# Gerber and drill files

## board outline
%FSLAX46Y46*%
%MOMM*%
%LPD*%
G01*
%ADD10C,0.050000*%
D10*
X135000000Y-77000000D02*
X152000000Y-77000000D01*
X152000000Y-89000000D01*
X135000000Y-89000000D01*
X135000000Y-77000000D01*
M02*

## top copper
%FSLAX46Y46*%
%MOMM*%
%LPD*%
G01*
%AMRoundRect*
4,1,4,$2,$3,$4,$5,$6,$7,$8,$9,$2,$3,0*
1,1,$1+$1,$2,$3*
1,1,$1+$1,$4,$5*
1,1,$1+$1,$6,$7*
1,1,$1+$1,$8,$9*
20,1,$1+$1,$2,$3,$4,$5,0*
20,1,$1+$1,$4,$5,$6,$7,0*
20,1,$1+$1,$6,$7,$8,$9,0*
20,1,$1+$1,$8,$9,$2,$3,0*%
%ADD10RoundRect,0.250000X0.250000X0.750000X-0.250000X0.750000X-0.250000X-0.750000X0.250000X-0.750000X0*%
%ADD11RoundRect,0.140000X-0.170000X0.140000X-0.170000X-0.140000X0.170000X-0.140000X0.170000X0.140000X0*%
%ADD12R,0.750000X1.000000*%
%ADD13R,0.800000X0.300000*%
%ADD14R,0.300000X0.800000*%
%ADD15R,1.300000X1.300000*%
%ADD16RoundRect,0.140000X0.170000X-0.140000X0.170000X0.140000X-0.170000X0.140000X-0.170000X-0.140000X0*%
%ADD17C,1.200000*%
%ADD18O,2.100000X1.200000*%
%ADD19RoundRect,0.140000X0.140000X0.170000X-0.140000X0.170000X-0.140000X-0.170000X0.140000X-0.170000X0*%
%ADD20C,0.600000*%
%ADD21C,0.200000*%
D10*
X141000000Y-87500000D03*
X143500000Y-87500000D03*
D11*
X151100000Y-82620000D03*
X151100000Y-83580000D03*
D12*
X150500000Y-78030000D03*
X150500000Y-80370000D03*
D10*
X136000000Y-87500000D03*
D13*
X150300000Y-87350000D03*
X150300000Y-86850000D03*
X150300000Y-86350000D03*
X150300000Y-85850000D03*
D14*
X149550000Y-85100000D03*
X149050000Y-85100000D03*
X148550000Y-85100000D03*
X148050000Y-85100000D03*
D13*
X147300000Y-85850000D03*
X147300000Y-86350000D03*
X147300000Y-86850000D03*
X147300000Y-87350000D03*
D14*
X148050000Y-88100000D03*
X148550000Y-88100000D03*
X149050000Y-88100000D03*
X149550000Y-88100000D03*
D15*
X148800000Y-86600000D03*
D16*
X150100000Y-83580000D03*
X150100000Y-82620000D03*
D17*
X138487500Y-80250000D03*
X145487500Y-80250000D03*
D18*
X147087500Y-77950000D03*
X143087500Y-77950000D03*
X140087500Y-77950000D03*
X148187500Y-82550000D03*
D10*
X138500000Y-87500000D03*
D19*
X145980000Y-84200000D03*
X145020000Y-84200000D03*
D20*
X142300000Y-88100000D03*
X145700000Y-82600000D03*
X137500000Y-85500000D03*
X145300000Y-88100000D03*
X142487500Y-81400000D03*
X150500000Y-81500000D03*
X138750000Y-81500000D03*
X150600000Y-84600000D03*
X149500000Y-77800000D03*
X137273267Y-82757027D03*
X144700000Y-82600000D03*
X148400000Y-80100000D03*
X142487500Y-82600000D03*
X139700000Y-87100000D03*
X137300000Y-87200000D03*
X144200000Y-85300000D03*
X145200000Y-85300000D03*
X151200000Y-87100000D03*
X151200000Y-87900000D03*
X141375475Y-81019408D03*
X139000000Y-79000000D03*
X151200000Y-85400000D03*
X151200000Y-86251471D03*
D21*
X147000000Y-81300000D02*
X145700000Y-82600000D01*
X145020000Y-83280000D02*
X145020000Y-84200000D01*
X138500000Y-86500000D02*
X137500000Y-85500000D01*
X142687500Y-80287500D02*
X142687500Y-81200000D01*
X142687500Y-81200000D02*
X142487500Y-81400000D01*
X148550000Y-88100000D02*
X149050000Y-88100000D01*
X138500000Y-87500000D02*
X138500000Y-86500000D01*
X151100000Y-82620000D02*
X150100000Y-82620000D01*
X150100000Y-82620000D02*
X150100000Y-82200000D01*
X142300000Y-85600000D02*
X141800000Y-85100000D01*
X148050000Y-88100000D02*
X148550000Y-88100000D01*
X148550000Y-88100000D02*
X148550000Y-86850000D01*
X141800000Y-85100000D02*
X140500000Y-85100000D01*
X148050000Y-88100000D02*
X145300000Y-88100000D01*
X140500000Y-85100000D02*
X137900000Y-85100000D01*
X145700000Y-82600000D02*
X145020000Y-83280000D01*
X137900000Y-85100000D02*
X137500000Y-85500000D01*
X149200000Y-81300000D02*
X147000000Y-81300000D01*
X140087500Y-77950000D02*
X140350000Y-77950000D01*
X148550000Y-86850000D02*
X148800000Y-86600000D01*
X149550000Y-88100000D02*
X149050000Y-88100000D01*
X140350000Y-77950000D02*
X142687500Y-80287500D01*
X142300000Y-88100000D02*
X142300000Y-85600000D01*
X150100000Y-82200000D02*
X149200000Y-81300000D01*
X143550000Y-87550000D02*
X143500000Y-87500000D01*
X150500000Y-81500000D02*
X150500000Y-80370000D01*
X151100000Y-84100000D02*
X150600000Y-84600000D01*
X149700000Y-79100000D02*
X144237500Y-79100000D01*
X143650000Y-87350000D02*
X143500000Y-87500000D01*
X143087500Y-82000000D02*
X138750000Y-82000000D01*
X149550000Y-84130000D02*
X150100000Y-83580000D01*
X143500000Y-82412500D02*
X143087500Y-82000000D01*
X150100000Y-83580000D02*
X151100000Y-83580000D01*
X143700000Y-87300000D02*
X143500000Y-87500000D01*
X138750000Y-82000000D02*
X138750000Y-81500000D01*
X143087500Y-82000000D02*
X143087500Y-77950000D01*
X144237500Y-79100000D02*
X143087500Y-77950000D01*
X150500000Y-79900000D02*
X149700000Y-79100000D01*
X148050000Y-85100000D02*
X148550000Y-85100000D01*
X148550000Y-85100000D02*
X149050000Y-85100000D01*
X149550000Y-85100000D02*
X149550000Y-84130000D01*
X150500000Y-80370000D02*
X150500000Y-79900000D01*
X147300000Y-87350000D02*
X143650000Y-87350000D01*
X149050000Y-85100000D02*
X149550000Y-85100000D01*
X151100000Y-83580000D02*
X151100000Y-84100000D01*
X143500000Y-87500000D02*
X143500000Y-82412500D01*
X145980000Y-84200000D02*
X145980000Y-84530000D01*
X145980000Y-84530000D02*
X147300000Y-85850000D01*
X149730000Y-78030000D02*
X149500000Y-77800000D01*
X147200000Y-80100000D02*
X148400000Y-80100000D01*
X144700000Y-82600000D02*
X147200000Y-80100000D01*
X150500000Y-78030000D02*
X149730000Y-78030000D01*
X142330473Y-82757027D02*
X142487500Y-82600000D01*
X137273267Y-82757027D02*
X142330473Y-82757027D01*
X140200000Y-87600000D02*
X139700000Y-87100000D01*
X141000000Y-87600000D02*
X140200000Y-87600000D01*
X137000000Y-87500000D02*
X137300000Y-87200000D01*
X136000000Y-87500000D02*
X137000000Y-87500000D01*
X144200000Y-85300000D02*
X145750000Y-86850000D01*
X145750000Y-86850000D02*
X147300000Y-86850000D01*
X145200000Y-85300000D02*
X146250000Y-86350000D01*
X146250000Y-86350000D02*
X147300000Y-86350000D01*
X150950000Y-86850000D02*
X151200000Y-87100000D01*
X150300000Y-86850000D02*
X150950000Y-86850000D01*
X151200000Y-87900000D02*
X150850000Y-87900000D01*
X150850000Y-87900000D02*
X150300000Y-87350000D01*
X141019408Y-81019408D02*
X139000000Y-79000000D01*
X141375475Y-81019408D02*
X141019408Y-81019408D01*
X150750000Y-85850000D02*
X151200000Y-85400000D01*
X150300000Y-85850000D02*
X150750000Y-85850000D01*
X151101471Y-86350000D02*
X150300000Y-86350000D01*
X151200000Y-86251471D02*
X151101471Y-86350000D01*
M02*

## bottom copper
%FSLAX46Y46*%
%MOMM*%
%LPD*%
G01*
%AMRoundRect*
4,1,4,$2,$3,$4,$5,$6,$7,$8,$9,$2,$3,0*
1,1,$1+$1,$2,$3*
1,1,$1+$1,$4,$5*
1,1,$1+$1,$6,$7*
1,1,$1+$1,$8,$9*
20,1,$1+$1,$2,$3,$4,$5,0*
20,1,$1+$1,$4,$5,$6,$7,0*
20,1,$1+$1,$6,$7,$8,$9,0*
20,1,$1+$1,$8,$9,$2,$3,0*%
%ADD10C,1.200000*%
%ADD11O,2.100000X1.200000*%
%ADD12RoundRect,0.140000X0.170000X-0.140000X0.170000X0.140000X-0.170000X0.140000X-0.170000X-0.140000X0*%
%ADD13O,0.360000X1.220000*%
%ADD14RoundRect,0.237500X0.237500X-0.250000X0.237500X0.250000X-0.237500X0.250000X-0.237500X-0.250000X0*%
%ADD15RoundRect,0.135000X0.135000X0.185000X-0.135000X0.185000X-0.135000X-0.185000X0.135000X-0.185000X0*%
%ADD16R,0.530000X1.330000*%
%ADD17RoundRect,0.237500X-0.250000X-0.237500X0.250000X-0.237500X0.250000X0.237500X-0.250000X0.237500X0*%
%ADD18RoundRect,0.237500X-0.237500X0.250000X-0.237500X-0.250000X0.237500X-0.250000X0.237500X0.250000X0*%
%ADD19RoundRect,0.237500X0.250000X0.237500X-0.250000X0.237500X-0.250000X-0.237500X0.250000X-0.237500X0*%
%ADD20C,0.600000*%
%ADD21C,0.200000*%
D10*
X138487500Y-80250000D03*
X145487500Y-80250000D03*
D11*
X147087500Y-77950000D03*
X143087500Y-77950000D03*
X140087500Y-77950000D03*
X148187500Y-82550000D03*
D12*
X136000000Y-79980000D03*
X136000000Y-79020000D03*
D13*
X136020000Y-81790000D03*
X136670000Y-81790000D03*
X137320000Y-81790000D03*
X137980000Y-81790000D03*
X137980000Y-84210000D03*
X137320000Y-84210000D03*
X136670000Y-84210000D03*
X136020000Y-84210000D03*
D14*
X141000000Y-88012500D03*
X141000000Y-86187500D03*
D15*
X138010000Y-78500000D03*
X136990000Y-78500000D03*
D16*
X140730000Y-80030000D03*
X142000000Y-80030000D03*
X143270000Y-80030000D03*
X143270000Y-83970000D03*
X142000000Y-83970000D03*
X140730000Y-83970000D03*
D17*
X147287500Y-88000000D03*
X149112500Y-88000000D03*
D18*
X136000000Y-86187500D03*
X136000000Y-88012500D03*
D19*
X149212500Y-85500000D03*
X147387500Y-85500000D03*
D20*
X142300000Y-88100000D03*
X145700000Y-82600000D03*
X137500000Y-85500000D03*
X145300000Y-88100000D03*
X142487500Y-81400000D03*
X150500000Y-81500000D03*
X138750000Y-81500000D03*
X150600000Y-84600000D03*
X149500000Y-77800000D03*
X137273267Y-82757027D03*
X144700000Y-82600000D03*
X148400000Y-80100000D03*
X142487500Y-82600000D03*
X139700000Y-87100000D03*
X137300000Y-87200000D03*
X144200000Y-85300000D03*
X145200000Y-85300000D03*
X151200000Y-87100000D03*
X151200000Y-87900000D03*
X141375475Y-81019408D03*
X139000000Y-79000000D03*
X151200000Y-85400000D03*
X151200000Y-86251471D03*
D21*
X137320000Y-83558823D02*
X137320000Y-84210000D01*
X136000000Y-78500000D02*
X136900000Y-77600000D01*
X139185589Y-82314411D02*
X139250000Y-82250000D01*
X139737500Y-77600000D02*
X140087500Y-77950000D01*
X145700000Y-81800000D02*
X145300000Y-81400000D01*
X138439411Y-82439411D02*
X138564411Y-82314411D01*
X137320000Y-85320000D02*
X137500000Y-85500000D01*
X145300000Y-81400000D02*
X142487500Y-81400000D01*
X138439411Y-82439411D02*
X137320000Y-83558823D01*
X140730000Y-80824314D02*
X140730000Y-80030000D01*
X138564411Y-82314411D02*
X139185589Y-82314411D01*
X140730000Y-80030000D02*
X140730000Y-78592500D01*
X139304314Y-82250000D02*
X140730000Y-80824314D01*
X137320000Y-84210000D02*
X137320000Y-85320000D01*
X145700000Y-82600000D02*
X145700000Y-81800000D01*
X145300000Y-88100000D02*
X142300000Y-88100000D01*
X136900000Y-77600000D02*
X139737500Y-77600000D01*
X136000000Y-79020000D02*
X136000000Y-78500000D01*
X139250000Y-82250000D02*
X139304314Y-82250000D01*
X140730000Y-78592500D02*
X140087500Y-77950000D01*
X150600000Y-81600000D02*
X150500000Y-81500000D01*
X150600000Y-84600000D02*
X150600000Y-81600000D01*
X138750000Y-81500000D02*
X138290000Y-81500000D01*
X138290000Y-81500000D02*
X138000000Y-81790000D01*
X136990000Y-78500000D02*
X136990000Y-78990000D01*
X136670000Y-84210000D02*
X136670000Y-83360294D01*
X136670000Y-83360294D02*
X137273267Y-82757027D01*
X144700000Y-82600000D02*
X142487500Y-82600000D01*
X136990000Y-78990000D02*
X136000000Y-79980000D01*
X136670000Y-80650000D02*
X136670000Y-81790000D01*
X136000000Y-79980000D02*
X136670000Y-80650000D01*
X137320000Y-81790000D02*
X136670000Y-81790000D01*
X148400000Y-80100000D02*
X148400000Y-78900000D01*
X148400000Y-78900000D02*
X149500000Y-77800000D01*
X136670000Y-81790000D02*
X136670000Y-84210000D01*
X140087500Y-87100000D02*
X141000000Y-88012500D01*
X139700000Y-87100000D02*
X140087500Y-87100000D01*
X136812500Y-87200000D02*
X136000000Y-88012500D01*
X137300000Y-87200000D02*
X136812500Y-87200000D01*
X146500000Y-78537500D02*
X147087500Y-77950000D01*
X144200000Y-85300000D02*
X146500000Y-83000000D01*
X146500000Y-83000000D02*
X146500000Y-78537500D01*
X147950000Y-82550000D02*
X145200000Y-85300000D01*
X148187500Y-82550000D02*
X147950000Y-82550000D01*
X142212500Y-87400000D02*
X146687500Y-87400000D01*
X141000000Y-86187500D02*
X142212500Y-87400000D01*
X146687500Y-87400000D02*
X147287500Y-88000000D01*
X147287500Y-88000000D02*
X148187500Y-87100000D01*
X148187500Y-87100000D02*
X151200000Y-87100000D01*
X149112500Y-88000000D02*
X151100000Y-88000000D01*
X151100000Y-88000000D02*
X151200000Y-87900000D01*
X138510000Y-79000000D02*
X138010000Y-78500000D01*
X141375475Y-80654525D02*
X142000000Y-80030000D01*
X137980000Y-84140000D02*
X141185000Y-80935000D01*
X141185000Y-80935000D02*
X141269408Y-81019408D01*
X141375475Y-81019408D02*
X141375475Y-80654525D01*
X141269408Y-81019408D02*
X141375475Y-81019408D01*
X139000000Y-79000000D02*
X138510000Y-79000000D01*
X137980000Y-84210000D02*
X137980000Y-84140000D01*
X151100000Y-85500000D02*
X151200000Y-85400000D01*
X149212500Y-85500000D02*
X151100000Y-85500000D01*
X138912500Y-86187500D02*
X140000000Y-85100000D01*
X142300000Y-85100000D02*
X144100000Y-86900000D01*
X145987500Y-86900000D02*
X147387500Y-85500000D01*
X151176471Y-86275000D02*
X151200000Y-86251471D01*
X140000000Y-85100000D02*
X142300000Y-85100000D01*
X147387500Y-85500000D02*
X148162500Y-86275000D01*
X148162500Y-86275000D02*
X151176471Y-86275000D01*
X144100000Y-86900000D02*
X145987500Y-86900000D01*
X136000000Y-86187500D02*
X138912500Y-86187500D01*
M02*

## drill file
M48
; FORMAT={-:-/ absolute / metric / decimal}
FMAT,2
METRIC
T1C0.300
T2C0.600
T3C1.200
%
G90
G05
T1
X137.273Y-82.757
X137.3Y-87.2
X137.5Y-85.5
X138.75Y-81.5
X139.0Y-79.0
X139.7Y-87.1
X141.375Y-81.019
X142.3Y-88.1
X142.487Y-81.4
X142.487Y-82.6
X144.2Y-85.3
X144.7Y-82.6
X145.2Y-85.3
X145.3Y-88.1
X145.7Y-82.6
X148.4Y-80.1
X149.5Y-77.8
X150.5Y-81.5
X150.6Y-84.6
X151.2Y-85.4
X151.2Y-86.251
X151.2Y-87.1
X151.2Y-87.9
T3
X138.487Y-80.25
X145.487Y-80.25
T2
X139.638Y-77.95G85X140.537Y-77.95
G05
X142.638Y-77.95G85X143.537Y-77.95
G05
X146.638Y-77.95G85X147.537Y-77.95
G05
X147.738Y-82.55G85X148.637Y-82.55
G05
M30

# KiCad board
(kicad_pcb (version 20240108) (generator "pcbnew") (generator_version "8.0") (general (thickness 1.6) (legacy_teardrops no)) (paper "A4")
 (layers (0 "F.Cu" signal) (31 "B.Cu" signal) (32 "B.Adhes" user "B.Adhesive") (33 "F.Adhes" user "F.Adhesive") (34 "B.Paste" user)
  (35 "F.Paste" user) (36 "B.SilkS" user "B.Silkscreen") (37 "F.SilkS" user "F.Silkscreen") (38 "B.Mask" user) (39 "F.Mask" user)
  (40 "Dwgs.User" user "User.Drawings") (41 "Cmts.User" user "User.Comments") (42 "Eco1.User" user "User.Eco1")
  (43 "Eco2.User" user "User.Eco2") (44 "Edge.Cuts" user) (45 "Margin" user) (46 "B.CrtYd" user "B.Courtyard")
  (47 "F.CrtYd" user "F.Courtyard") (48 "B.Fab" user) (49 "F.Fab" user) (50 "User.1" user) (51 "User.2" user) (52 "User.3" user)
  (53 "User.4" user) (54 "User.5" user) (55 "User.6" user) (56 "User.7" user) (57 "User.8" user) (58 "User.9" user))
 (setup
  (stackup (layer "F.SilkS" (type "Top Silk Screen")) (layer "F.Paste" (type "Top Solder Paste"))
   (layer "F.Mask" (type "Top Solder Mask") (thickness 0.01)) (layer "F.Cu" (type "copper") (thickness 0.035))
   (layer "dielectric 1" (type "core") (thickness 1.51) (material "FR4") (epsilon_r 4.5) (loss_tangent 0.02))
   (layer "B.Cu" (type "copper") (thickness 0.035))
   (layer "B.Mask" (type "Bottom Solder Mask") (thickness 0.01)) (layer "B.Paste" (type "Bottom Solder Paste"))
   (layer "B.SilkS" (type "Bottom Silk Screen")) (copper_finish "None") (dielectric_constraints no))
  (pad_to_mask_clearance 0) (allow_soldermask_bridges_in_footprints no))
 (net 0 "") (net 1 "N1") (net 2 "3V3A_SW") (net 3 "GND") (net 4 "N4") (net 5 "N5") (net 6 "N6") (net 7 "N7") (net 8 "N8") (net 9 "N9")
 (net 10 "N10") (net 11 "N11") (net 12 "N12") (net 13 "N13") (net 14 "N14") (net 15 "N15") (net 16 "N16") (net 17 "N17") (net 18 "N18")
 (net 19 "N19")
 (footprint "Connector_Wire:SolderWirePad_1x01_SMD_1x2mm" (layer "F.Cu") (at 141 87.5 180)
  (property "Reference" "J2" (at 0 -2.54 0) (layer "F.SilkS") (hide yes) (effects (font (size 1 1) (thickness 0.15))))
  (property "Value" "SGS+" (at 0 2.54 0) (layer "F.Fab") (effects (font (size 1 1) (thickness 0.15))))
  (pad "1" smd roundrect (at 0 0 180) (size 1 2) (layers "F.Cu" "F.Paste" "F.Mask") (roundrect_rratio 0.25) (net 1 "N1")))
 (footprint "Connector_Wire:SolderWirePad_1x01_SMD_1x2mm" (layer "F.Cu") (at 143.5 87.5 180)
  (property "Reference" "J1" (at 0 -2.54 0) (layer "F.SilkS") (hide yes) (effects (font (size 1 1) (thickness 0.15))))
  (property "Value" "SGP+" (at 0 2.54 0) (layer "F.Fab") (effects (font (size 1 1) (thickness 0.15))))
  (pad "1" smd roundrect (at 0 0 180) (size 1 2) (layers "F.Cu" "F.Paste" "F.Mask") (roundrect_rratio 0.25) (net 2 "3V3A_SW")))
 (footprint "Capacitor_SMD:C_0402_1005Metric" (layer "F.Cu") (at 151.1 83.1 -90)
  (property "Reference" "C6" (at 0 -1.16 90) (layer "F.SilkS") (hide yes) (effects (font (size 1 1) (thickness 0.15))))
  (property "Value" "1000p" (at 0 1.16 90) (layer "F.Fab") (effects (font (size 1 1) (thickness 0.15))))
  (pad "1" smd roundrect (at -0.48 0 270) (size 0.56 0.62) (layers "F.Cu" "F.Paste" "F.Mask") (roundrect_rratio 0.25) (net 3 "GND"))
  (pad "2" smd roundrect (at 0.48 0 270) (size 0.56 0.62) (layers "F.Cu" "F.Paste" "F.Mask") (roundrect_rratio 0.25) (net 2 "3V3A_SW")))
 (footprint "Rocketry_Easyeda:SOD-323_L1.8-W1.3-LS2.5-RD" (layer "F.Cu") (at 150.5 79.2 -90)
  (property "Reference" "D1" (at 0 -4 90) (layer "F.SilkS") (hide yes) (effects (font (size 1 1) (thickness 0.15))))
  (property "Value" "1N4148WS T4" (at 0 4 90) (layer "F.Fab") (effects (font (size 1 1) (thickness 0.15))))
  (pad "1" smd rect (at -1.17 0 270) (size 1 0.75) (layers "F.Cu" "F.Paste" "F.Mask") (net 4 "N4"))
  (pad "2" smd rect (at 1.17 0 270) (size 1 0.75) (layers "F.Cu" "F.Paste" "F.Mask") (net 2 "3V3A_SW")))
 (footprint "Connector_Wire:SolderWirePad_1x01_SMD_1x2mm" (layer "F.Cu") (at 136 87.5 180)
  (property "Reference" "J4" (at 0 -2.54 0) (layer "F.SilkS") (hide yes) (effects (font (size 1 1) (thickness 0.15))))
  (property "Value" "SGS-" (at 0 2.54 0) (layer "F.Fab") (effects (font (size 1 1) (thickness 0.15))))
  (pad "1" smd roundrect (at 0 0 180) (size 1 2) (layers "F.Cu" "F.Paste" "F.Mask") (roundrect_rratio 0.25) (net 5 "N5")))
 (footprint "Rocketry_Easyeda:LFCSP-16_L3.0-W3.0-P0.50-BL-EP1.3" (layer "F.Cu") (at 148.8 86.6 90)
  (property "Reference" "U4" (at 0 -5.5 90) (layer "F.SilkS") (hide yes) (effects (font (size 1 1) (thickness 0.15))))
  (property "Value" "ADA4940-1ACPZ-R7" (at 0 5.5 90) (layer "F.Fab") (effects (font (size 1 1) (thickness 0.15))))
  (pad "1" smd rect (at -0.75 1.5 270) (size 0.3 0.8) (layers "F.Cu" "F.Paste" "F.Mask") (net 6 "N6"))
  (pad "2" smd rect (at -0.25 1.5 270) (size 0.3 0.8) (layers "F.Cu" "F.Paste" "F.Mask") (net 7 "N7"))
  (pad "3" smd rect (at 0.25 1.5 270) (size 0.3 0.8) (layers "F.Cu" "F.Paste" "F.Mask") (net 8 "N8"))
  (pad "4" smd rect (at 0.75 1.5 270) (size 0.3 0.8) (layers "F.Cu" "F.Paste" "F.Mask") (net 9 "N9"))
  (pad "5" smd rect (at 1.5 0.75 180) (size 0.3 0.8) (layers "F.Cu" "F.Paste" "F.Mask") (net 2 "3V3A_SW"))
  (pad "6" smd rect (at 1.5 0.25 180) (size 0.3 0.8) (layers "F.Cu" "F.Paste" "F.Mask") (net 2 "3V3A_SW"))
  (pad "7" smd rect (at 1.5 -0.25 180) (size 0.3 0.8) (layers "F.Cu" "F.Paste" "F.Mask") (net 2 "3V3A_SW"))
  (pad "8" smd rect (at 1.5 -0.75 180) (size 0.3 0.8) (layers "F.Cu" "F.Paste" "F.Mask") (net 2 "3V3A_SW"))
  (pad "9" smd rect (at 0.75 -1.5 270) (size 0.3 0.8) (layers "F.Cu" "F.Paste" "F.Mask") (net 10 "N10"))
  (pad "10" smd rect (at 0.25 -1.5 270) (size 0.3 0.8) (layers "F.Cu" "F.Paste" "F.Mask") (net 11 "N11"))
  (pad "11" smd rect (at -0.25 -1.5 270) (size 0.3 0.8) (layers "F.Cu" "F.Paste" "F.Mask") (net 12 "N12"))
  (pad "12" smd rect (at -0.75 -1.5 270) (size 0.3 0.8) (layers "F.Cu" "F.Paste" "F.Mask") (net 2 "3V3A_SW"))
  (pad "13" smd rect (at -1.5 -0.75 180) (size 0.3 0.8) (layers "F.Cu" "F.Paste" "F.Mask") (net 3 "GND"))
  (pad "14" smd rect (at -1.5 -0.25 180) (size 0.3 0.8) (layers "F.Cu" "F.Paste" "F.Mask") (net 3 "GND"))
  (pad "15" smd rect (at -1.5 0.25 180) (size 0.3 0.8) (layers "F.Cu" "F.Paste" "F.Mask") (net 3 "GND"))
  (pad "16" smd rect (at -1.5 0.75 180) (size 0.3 0.8) (layers "F.Cu" "F.Paste" "F.Mask") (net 3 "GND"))
  (pad "17" smd rect (at 0 0 270) (size 1.3 1.3) (layers "F.Cu" "F.Paste" "F.Mask") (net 3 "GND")))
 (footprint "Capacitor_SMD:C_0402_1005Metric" (layer "F.Cu") (at 150.1 83.1 90)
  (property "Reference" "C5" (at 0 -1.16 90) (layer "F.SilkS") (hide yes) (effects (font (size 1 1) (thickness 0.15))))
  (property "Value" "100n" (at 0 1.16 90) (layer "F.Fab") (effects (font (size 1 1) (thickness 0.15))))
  (pad "1" smd roundrect (at -0.48 0 90) (size 0.56 0.62) (layers "F.Cu" "F.Paste" "F.Mask") (roundrect_rratio 0.25) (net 2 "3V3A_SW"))
  (pad "2" smd roundrect (at 0.48 0 90) (size 0.56 0.62) (layers "F.Cu" "F.Paste" "F.Mask") (roundrect_rratio 0.25) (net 3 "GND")))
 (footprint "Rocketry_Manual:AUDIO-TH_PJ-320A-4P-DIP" (layer "F.Cu") (at 144.1375 80.25)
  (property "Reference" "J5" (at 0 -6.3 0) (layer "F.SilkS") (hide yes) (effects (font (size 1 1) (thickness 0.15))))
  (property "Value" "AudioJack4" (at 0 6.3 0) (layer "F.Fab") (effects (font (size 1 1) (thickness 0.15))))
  (pad "" thru_hole circle (at -5.65 0) (size 1.2 1.2) (drill 1.2) (layers "*.Cu" "*.Mask") (remove_unused_layers no))
  (pad "" thru_hole circle (at 1.35 0) (size 1.2 1.2) (drill 1.2) (layers "*.Cu" "*.Mask") (remove_unused_layers no))
  (pad "R1" thru_hole oval (at 2.95 -2.3 90) (size 1.2 2.1) (drill oval 0.599999 1.499997) (layers "*.Cu" "*.Mask")
   (remove_unused_layers no) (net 12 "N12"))
  (pad "R2" thru_hole oval (at -1.05 -2.3 90) (size 1.2 2.1) (drill oval 0.599999 1.499997) (layers "*.Cu" "*.Mask")
   (remove_unused_layers no) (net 2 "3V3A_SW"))
  (pad "S" thru_hole oval (at -4.05 -2.3 90) (size 1.2 2.1) (drill oval 0.599999 1.499997) (layers "*.Cu" "*.Mask")
   (remove_unused_layers no) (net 3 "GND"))
  (pad "T" thru_hole oval (at 4.05 2.3 90) (size 1.2 2.1) (drill oval 0.599999 1.499997) (layers "*.Cu" "*.Mask") (remove_unused_layers no)
   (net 11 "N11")))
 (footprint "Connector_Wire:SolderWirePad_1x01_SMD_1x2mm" (layer "F.Cu") (at 138.5 87.5 180)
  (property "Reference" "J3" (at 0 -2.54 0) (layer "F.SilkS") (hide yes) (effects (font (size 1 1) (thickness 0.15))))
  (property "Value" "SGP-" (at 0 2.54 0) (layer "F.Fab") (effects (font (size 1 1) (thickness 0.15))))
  (pad "1" smd roundrect (at 0 0 180) (size 1 2) (layers "F.Cu" "F.Paste" "F.Mask") (roundrect_rratio 0.25) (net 3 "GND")))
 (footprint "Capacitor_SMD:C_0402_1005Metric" (layer "F.Cu") (at 145.5 84.2 180)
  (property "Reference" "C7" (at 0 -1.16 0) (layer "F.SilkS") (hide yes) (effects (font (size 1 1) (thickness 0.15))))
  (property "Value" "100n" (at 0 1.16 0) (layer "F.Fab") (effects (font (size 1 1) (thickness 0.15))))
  (pad "1" smd roundrect (at -0.48 0 180) (size 0.56 0.62) (layers "F.Cu" "F.Paste" "F.Mask") (roundrect_rratio 0.25) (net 10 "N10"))
  (pad "2" smd roundrect (at 0.48 0 180) (size 0.56 0.62) (layers "F.Cu" "F.Paste" "F.Mask") (roundrect_rratio 0.25) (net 3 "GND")))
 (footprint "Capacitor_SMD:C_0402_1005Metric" (layer "B.Cu") (at 136 79.5 90)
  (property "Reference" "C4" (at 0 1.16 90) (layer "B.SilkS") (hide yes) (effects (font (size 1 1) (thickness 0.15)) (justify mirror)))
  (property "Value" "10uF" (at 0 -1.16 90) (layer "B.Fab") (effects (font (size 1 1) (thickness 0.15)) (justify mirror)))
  (pad "1" smd roundrect (at -0.48 0 90) (size 0.56 0.62) (layers "B.Cu" "B.Paste" "B.Mask") (roundrect_rratio 0.25) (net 4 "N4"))
  (pad "2" smd roundrect (at 0.48 0 90) (size 0.56 0.62) (layers "B.Cu" "B.Paste" "B.Mask") (roundrect_rratio 0.25) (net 3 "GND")))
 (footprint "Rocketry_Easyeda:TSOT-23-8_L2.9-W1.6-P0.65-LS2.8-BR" (layer "B.Cu") (at 137 83 90)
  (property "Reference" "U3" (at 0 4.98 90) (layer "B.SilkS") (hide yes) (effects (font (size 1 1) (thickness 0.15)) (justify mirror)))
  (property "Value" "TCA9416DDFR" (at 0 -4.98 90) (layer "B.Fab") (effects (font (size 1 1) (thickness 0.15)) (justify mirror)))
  (pad "1" smd oval (at 1.21 -0.98 90) (size 1.22 0.36) (layers "B.Cu" "B.Paste" "B.Mask") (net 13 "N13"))
  (pad "2" smd oval (at 1.21 -0.33 90) (size 1.22 0.36) (layers "B.Cu" "B.Paste" "B.Mask") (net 4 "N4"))
  (pad "3" smd oval (at 1.21 0.32 90) (size 1.22 0.36) (layers "B.Cu" "B.Paste" "B.Mask") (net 4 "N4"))
  (pad "4" smd oval (at 1.21 0.98 90) (size 1.22 0.36) (layers "B.Cu" "B.Paste" "B.Mask") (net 2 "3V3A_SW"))
  (pad "5" smd oval (at -1.21 0.98 90) (size 1.22 0.36) (layers "B.Cu" "B.Paste" "B.Mask") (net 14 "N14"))
  (pad "6" smd oval (at -1.21 0.32 90) (size 1.22 0.36) (layers "B.Cu" "B.Paste" "B.Mask") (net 3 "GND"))
  (pad "7" smd oval (at -1.21 -0.33 90) (size 1.22 0.36) (layers "B.Cu" "B.Paste" "B.Mask") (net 4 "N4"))
  (pad "8" smd oval (at -1.21 -0.98 90) (size 1.22 0.36) (layers "B.Cu" "B.Paste" "B.Mask") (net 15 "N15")))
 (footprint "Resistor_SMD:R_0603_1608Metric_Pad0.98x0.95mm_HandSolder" (layer "B.Cu") (at 141 87.1 90)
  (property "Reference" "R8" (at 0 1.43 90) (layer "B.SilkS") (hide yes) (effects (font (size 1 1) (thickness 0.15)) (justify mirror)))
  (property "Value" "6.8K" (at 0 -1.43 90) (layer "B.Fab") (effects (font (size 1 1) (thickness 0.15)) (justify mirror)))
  (pad "1" smd roundrect (at -0.9125 0 90) (size 0.975 0.95) (layers "B.Cu" "B.Paste" "B.Mask") (roundrect_rratio 0.25) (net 1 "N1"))
  (pad "2" smd roundrect (at 0.9125 0 90) (size 0.975 0.95) (layers "B.Cu" "B.Paste" "B.Mask") (roundrect_rratio 0.25) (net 7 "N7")))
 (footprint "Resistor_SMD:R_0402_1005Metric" (layer "B.Cu") (at 137.5 78.5 180)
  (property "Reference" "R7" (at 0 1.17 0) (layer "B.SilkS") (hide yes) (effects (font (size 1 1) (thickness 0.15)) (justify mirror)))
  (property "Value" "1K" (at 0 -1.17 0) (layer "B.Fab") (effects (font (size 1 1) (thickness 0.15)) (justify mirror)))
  (pad "1" smd roundrect (at -0.51 0 180) (size 0.54 0.64) (layers "B.Cu" "B.Paste" "B.Mask") (roundrect_rratio 0.25) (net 14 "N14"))
  (pad "2" smd roundrect (at 0.51 0 180) (size 0.54 0.64) (layers "B.Cu" "B.Paste" "B.Mask") (roundrect_rratio 0.25) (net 4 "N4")))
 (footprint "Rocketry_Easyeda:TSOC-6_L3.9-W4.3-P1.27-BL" (layer "B.Cu") (at 142 82)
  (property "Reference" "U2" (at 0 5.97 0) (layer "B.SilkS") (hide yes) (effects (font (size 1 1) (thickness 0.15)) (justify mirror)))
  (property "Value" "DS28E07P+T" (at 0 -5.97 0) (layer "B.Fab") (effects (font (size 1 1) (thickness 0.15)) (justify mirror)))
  (pad "1" smd rect (at -1.27 -1.97) (size 0.53 1.33) (layers "B.Cu" "B.Paste" "B.Mask") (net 3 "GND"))
  (pad "2" smd rect (at 0 -1.97) (size 0.53 1.33) (layers "B.Cu" "B.Paste" "B.Mask") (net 14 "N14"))
  (pad "3" smd rect (at 1.27 -1.97) (size 0.53 1.33) (layers "B.Cu" "B.Paste" "B.Mask") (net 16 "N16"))
  (pad "4" smd rect (at 1.27 1.97) (size 0.53 1.33) (layers "B.Cu" "B.Paste" "B.Mask") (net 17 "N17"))
  (pad "5" smd rect (at 0 1.97) (size 0.53 1.33) (layers "B.Cu" "B.Paste" "B.Mask") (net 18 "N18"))
  (pad "6" smd rect (at -1.27 1.97) (size 0.53 1.33) (layers "B.Cu" "B.Paste" "B.Mask") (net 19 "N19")))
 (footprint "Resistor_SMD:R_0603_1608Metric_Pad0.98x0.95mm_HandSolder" (layer "B.Cu") (at 148.2 88)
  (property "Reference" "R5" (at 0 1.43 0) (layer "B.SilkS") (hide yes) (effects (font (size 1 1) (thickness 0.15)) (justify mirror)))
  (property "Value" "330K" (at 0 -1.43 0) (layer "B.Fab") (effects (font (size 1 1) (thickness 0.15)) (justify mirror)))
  (pad "1" smd roundrect (at -0.9125 0) (size 0.975 0.95) (layers "B.Cu" "B.Paste" "B.Mask") (roundrect_rratio 0.25) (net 7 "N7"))
  (pad "2" smd roundrect (at 0.9125 0) (size 0.975 0.95) (layers "B.Cu" "B.Paste" "B.Mask") (roundrect_rratio 0.25) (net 6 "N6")))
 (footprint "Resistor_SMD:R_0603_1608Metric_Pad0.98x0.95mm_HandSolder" (layer "B.Cu") (at 136 87.1 -90)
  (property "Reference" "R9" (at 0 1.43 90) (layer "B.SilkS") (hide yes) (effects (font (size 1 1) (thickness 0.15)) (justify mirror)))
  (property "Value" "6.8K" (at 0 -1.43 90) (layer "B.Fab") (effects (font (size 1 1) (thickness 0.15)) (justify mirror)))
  (pad "1" smd roundrect (at -0.9125 0 270) (size 0.975 0.95) (layers "B.Cu" "B.Paste" "B.Mask") (roundrect_rratio 0.25) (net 8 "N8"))
  (pad "2" smd roundrect (at 0.9125 0 270) (size 0.975 0.95) (layers "B.Cu" "B.Paste" "B.Mask") (roundrect_rratio 0.25) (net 5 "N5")))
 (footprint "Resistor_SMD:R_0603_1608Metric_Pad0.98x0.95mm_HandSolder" (layer "B.Cu") (at 148.3 85.5 180)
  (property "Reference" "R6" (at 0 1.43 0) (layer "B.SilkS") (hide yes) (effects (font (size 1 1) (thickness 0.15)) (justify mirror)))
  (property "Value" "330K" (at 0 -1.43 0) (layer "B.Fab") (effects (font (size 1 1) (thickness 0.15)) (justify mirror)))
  (pad "1" smd roundrect (at -0.9125 0 180) (size 0.975 0.95) (layers "B.Cu" "B.Paste" "B.Mask") (roundrect_rratio 0.25) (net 9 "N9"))
  (pad "2" smd roundrect (at 0.9125 0 180) (size 0.975 0.95) (layers "B.Cu" "B.Paste" "B.Mask") (roundrect_rratio 0.25) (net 8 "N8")))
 (gr_rect (start 135 77) (end 152 89) (stroke (width 0.05) (type default)) (fill none) (layer "Edge.Cuts"))
 (segment (start 147 81.3) (end 145.7 82.6) (width 0.2) (layer "F.Cu") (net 3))
 (segment (start 145.02 83.28) (end 145.02 84.2) (width 0.2) (layer "F.Cu") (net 3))
 (segment (start 138.5 86.5) (end 137.5 85.5) (width 0.2) (layer "F.Cu") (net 3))
 (segment (start 142.6875 80.2875) (end 142.6875 81.2) (width 0.2) (layer "F.Cu") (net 3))
 (segment (start 142.6875 81.2) (end 142.4875 81.4) (width 0.2) (layer "F.Cu") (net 3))
 (segment (start 148.55 88.1) (end 149.05 88.1) (width 0.2) (layer "F.Cu") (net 3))
 (segment (start 138.5 87.5) (end 138.5 86.5) (width 0.2) (layer "F.Cu") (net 3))
 (segment (start 151.1 82.62) (end 150.1 82.62) (width 0.2) (layer "F.Cu") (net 3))
 (segment (start 150.1 82.62) (end 150.1 82.2) (width 0.2) (layer "F.Cu") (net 3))
 (segment (start 142.3 85.6) (end 141.8 85.1) (width 0.2) (layer "F.Cu") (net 3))
 (segment (start 148.05 88.1) (end 148.55 88.1) (width 0.2) (layer "F.Cu") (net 3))
 (segment (start 148.55 88.1) (end 148.55 86.85) (width 0.2) (layer "F.Cu") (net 3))
 (segment (start 141.8 85.1) (end 140.5 85.1) (width 0.2) (layer "F.Cu") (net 3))
 (segment (start 148.05 88.1) (end 145.3 88.1) (width 0.2) (layer "F.Cu") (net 3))
 (segment (start 140.5 85.1) (end 137.9 85.1) (width 0.2) (layer "F.Cu") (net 3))
 (segment (start 145.7 82.6) (end 145.02 83.28) (width 0.2) (layer "F.Cu") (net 3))
 (segment (start 137.9 85.1) (end 137.5 85.5) (width 0.2) (layer "F.Cu") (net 3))
 (segment (start 149.2 81.3) (end 147 81.3) (width 0.2) (layer "F.Cu") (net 3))
 (segment (start 140.0875 77.95) (end 140.35 77.95) (width 0.2) (layer "F.Cu") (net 3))
 (segment (start 148.55 86.85) (end 148.8 86.6) (width 0.2) (layer "F.Cu") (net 3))
 (segment (start 149.55 88.1) (end 149.05 88.1) (width 0.2) (layer "F.Cu") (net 3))
 (segment (start 140.35 77.95) (end 142.6875 80.2875) (width 0.2) (layer "F.Cu") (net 3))
 (segment (start 142.3 88.1) (end 142.3 85.6) (width 0.2) (layer "F.Cu") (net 3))
 (segment (start 150.1 82.2) (end 149.2 81.3) (width 0.2) (layer "F.Cu") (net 3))
 (via (at 142.3 88.1) (size 0.6) (drill 0.3) (layers "F.Cu" "B.Cu") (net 3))
 (via (at 145.7 82.6) (size 0.6) (drill 0.3) (layers "F.Cu" "B.Cu") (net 3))
 (via (at 137.5 85.5) (size 0.6) (drill 0.3) (layers "F.Cu" "B.Cu") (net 3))
 (via (at 145.3 88.1) (size 0.6) (drill 0.3) (layers "F.Cu" "B.Cu") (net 3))
 (via (at 142.4875 81.4) (size 0.6) (drill 0.3) (layers "F.Cu" "B.Cu") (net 3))
 (segment (start 137.32 83.558823) (end 137.32 84.21) (width 0.2) (layer "B.Cu") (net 3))
 (segment (start 136 78.5) (end 136.9 77.6) (width 0.2) (layer "B.Cu") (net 3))
 (segment (start 139.185589 82.314411) (end 139.25 82.25) (width 0.2) (layer "B.Cu") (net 3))
 (segment (start 139.7375 77.6) (end 140.0875 77.95) (width 0.2) (layer "B.Cu") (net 3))
 (segment (start 145.7 81.8) (end 145.3 81.4) (width 0.2) (layer "B.Cu") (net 3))
 (segment (start 138.439411 82.439411) (end 138.564411 82.314411) (width 0.2) (layer "B.Cu") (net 3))
 (segment (start 137.32 85.32) (end 137.5 85.5) (width 0.2) (layer "B.Cu") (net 3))
 (segment (start 145.3 81.4) (end 142.4875 81.4) (width 0.2) (layer "B.Cu") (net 3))
 (segment (start 138.439411 82.439411) (end 137.32 83.558823) (width 0.2) (layer "B.Cu") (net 3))
 (segment (start 140.73 80.824314) (end 140.73 80.03) (width 0.2) (layer "B.Cu") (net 3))
 (segment (start 138.564411 82.314411) (end 139.185589 82.314411) (width 0.2) (layer "B.Cu") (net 3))
 (segment (start 140.73 80.03) (end 140.73 78.5925) (width 0.2) (layer "B.Cu") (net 3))
 (segment (start 139.304314 82.25) (end 140.73 80.824314) (width 0.2) (layer "B.Cu") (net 3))
 (segment (start 137.32 84.21) (end 137.32 85.32) (width 0.2) (layer "B.Cu") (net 3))
 (segment (start 145.7 82.6) (end 145.7 81.8) (width 0.2) (layer "B.Cu") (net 3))
 (segment (start 145.3 88.1) (end 142.3 88.1) (width 0.2) (layer "B.Cu") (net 3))
 (segment (start 136.9 77.6) (end 139.7375 77.6) (width 0.2) (layer "B.Cu") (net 3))
 (segment (start 136 79.02) (end 136 78.5) (width 0.2) (layer "B.Cu") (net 3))
 (segment (start 139.25 82.25) (end 139.304314 82.25) (width 0.2) (layer "B.Cu") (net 3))
 (segment (start 140.73 78.5925) (end 140.0875 77.95) (width 0.2) (layer "B.Cu") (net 3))
 (segment (start 143.55 87.55) (end 143.5 87.5) (width 0.2) (layer "F.Cu") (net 2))
 (segment (start 150.5 81.5) (end 150.5 80.37) (width 0.2) (layer "F.Cu") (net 2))
 (segment (start 151.1 84.1) (end 150.6 84.6) (width 0.2) (layer "F.Cu") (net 2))
 (segment (start 149.7 79.1) (end 144.2375 79.1) (width 0.2) (layer "F.Cu") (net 2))
 (segment (start 143.65 87.35) (end 143.5 87.5) (width 0.2) (layer "F.Cu") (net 2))
 (segment (start 143.0875 82) (end 138.75 82) (width 0.2) (layer "F.Cu") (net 2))
 (segment (start 149.55 84.13) (end 150.1 83.58) (width 0.2) (layer "F.Cu") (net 2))
 (segment (start 143.5 82.4125) (end 143.0875 82) (width 0.2) (layer "F.Cu") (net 2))
 (segment (start 150.1 83.58) (end 151.1 83.58) (width 0.2) (layer "F.Cu") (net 2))
 (segment (start 143.7 87.3) (end 143.5 87.5) (width 0.2) (layer "F.Cu") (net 2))
 (segment (start 138.75 82) (end 138.75 81.5) (width 0.2) (layer "F.Cu") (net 2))
 (segment (start 143.0875 82) (end 143.0875 77.95) (width 0.2) (layer "F.Cu") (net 2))
 (segment (start 144.2375 79.1) (end 143.0875 77.95) (width 0.2) (layer "F.Cu") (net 2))
 (segment (start 150.5 79.9) (end 149.7 79.1) (width 0.2) (layer "F.Cu") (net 2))
 (segment (start 148.05 85.1) (end 148.55 85.1) (width 0.2) (layer "F.Cu") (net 2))
 (segment (start 148.55 85.1) (end 149.05 85.1) (width 0.2) (layer "F.Cu") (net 2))
 (segment (start 149.55 85.1) (end 149.55 84.13) (width 0.2) (layer "F.Cu") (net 2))
 (segment (start 150.5 80.37) (end 150.5 79.9) (width 0.2) (layer "F.Cu") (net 2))
 (segment (start 147.3 87.35) (end 143.65 87.35) (width 0.2) (layer "F.Cu") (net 2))
 (segment (start 149.05 85.1) (end 149.55 85.1) (width 0.2) (layer "F.Cu") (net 2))
 (segment (start 151.1 83.58) (end 151.1 84.1) (width 0.2) (layer "F.Cu") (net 2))
 (segment (start 143.5 87.5) (end 143.5 82.4125) (width 0.2) (layer "F.Cu") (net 2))
 (via (at 150.5 81.5) (size 0.6) (drill 0.3) (layers "F.Cu" "B.Cu") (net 2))
 (via (at 138.75 81.5) (size 0.6) (drill 0.3) (layers "F.Cu" "B.Cu") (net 2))
 (via (at 150.6 84.6) (size 0.6) (drill 0.3) (layers "F.Cu" "B.Cu") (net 2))
 (segment (start 150.6 81.6) (end 150.5 81.5) (width 0.2) (layer "B.Cu") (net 2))
 (segment (start 150.6 84.6) (end 150.6 81.6) (width 0.2) (layer "B.Cu") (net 2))
 (segment (start 138.75 81.5) (end 138.29 81.5) (width 0.2) (layer "B.Cu") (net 2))
 (segment (start 138.29 81.5) (end 138 81.79) (width 0.2) (layer "B.Cu") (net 2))
 (segment (start 145.98 84.2) (end 145.98 84.53) (width 0.2) (layer "F.Cu") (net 10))
 (segment (start 145.98 84.53) (end 147.3 85.85) (width 0.2) (layer "F.Cu") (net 10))
 (segment (start 149.73 78.03) (end 149.5 77.8) (width 0.2) (layer "F.Cu") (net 4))
 (segment (start 147.2 80.1) (end 148.4 80.1) (width 0.2) (layer "F.Cu") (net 4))
 (segment (start 144.7 82.6) (end 147.2 80.1) (width 0.2) (layer "F.Cu") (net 4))
 (segment (start 150.5 78.03) (end 149.73 78.03) (width 0.2) (layer "F.Cu") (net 4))
 (segment (start 142.330473 82.757027) (end 142.4875 82.6) (width 0.2) (layer "F.Cu") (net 4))
 (segment (start 137.273267 82.757027) (end 142.330473 82.757027) (width 0.2) (layer "F.Cu") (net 4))
 (via (at 149.5 77.8) (size 0.6) (drill 0.3) (layers "F.Cu" "B.Cu") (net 4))
 (via (at 137.273267 82.757027) (size 0.6) (drill 0.3) (layers "F.Cu" "B.Cu") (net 4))
 (via (at 144.7 82.6) (size 0.6) (drill 0.3) (layers "F.Cu" "B.Cu") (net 4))
 (via (at 148.4 80.1) (size 0.6) (drill 0.3) (layers "F.Cu" "B.Cu") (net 4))
 (via (at 142.4875 82.6) (size 0.6) (drill 0.3) (layers "F.Cu" "B.Cu") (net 4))
 (segment (start 136.99 78.5) (end 136.99 78.99) (width 0.2) (layer "B.Cu") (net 4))
 (segment (start 136.67 84.21) (end 136.67 83.360294) (width 0.2) (layer "B.Cu") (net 4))
 (segment (start 136.67 83.360294) (end 137.273267 82.757027) (width 0.2) (layer "B.Cu") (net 4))
 (segment (start 144.7 82.6) (end 142.4875 82.6) (width 0.2) (layer "B.Cu") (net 4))
 (segment (start 136.99 78.99) (end 136 79.98) (width 0.2) (layer "B.Cu") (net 4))
 (segment (start 136.67 80.65) (end 136.67 81.79) (width 0.2) (layer "B.Cu") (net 4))
 (segment (start 136 79.98) (end 136.67 80.65) (width 0.2) (layer "B.Cu") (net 4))
 (segment (start 137.32 81.79) (end 136.67 81.79) (width 0.2) (layer "B.Cu") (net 4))
 (segment (start 148.4 80.1) (end 148.4 78.9) (width 0.2) (layer "B.Cu") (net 4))
 (segment (start 148.4 78.9) (end 149.5 77.8) (width 0.2) (layer "B.Cu") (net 4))
 (segment (start 136.67 81.79) (end 136.67 84.21) (width 0.2) (layer "B.Cu") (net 4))
 (segment (start 140.2 87.6) (end 139.7 87.1) (width 0.2) (layer "F.Cu") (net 1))
 (segment (start 141 87.6) (end 140.2 87.6) (width 0.2) (layer "F.Cu") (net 1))
 (via (at 139.7 87.1) (size 0.6) (drill 0.3) (layers "F.Cu" "B.Cu") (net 1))
 (segment (start 140.0875 87.1) (end 141 88.0125) (width 0.2) (layer "B.Cu") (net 1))
 (segment (start 139.7 87.1) (end 140.0875 87.1) (width 0.2) (layer "B.Cu") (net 1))
 (segment (start 137 87.5) (end 137.3 87.2) (width 0.2) (layer "F.Cu") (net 5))
 (segment (start 136 87.5) (end 137 87.5) (width 0.2) (layer "F.Cu") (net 5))
 (via (at 137.3 87.2) (size 0.6) (drill 0.3) (layers "F.Cu" "B.Cu") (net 5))
 (segment (start 136.8125 87.2) (end 136 88.0125) (width 0.2) (layer "B.Cu") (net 5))
 (segment (start 137.3 87.2) (end 136.8125 87.2) (width 0.2) (layer "B.Cu") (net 5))
 (segment (start 144.2 85.3) (end 145.75 86.85) (width 0.2) (layer "F.Cu") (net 12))
 (segment (start 145.75 86.85) (end 147.3 86.85) (width 0.2) (layer "F.Cu") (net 12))
 (via (at 144.2 85.3) (size 0.6) (drill 0.3) (layers "F.Cu" "B.Cu") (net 12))
 (segment (start 146.5 78.5375) (end 147.0875 77.95) (width 0.2) (layer "B.Cu") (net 12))
 (segment (start 144.2 85.3) (end 146.5 83) (width 0.2) (layer "B.Cu") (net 12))
 (segment (start 146.5 83) (end 146.5 78.5375) (width 0.2) (layer "B.Cu") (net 12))
 (segment (start 145.2 85.3) (end 146.25 86.35) (width 0.2) (layer "F.Cu") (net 11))
 (segment (start 146.25 86.35) (end 147.3 86.35) (width 0.2) (layer "F.Cu") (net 11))
 (via (at 145.2 85.3) (size 0.6) (drill 0.3) (layers "F.Cu" "B.Cu") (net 11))
 (segment (start 147.95 82.55) (end 145.2 85.3) (width 0.2) (layer "B.Cu") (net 11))
 (segment (start 148.1875 82.55) (end 147.95 82.55) (width 0.2) (layer "B.Cu") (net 11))
 (segment (start 150.95 86.85) (end 151.2 87.1) (width 0.2) (layer "F.Cu") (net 7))
 (segment (start 150.3 86.85) (end 150.95 86.85) (width 0.2) (layer "F.Cu") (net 7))
 (via (at 151.2 87.1) (size 0.6) (drill 0.3) (layers "F.Cu" "B.Cu") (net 7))
 (segment (start 142.2125 87.4) (end 146.6875 87.4) (width 0.2) (layer "B.Cu") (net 7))
 (segment (start 141 86.1875) (end 142.2125 87.4) (width 0.2) (layer "B.Cu") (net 7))
 (segment (start 146.6875 87.4) (end 147.2875 88) (width 0.2) (layer "B.Cu") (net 7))
 (segment (start 147.2875 88) (end 148.1875 87.1) (width 0.2) (layer "B.Cu") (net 7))
 (segment (start 148.1875 87.1) (end 151.2 87.1) (width 0.2) (layer "B.Cu") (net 7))
 (segment (start 151.2 87.9) (end 150.85 87.9) (width 0.2) (layer "F.Cu") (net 6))
 (segment (start 150.85 87.9) (end 150.3 87.35) (width 0.2) (layer "F.Cu") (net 6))
 (via (at 151.2 87.9) (size 0.6) (drill 0.3) (layers "F.Cu" "B.Cu") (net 6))
 (segment (start 149.1125 88) (end 151.1 88) (width 0.2) (layer "B.Cu") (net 6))
 (segment (start 151.1 88) (end 151.2 87.9) (width 0.2) (layer "B.Cu") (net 6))
 (segment (start 141.019408 81.019408) (end 139 79) (width 0.2) (layer "F.Cu") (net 14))
 (segment (start 141.375475 81.019408) (end 141.019408 81.019408) (width 0.2) (layer "F.Cu") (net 14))
 (via (at 141.375475 81.019408) (size 0.6) (drill 0.3) (layers "F.Cu" "B.Cu") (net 14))
 (via (at 139 79) (size 0.6) (drill 0.3) (layers "F.Cu" "B.Cu") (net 14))
 (segment (start 138.51 79) (end 138.01 78.5) (width 0.2) (layer "B.Cu") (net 14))
 (segment (start 141.375475 80.654525) (end 142 80.03) (width 0.2) (layer "B.Cu") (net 14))
 (segment (start 137.98 84.14) (end 141.185 80.935) (width 0.2) (layer "B.Cu") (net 14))
 (segment (start 141.185 80.935) (end 141.269408 81.019408) (width 0.2) (layer "B.Cu") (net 14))
 (segment (start 141.375475 81.019408) (end 141.375475 80.654525) (width 0.2) (layer "B.Cu") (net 14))
 (segment (start 141.269408 81.019408) (end 141.375475 81.019408) (width 0.2) (layer "B.Cu") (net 14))
 (segment (start 139 79) (end 138.51 79) (width 0.2) (layer "B.Cu") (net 14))
 (segment (start 137.98 84.21) (end 137.98 84.14) (width 0.2) (layer "B.Cu") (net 14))
 (segment (start 150.75 85.85) (end 151.2 85.4) (width 0.2) (layer "F.Cu") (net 9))
 (segment (start 150.3 85.85) (end 150.75 85.85) (width 0.2) (layer "F.Cu") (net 9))
 (via (at 151.2 85.4) (size 0.6) (drill 0.3) (layers "F.Cu" "B.Cu") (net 9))
 (segment (start 151.1 85.5) (end 151.2 85.4) (width 0.2) (layer "B.Cu") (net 9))
 (segment (start 149.2125 85.5) (end 151.1 85.5) (width 0.2) (layer "B.Cu") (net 9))
 (segment (start 151.101471 86.35) (end 150.3 86.35) (width 0.2) (layer "F.Cu") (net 8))
 (segment (start 151.2 86.251471) (end 151.101471 86.35) (width 0.2) (layer "F.Cu") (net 8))
 (via (at 151.2 86.251471) (size 0.6) (drill 0.3) (layers "F.Cu" "B.Cu") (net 8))
 (segment (start 138.9125 86.1875) (end 140 85.1) (width 0.2) (layer "B.Cu") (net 8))
 (segment (start 142.3 85.1) (end 144.1 86.9) (width 0.2) (layer "B.Cu") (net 8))
 (segment (start 145.9875 86.9) (end 147.3875 85.5) (width 0.2) (layer "B.Cu") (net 8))
 (segment (start 151.176471 86.275) (end 151.2 86.251471) (width 0.2) (layer "B.Cu") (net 8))
 (segment (start 140 85.1) (end 142.3 85.1) (width 0.2) (layer "B.Cu") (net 8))
 (segment (start 147.3875 85.5) (end 148.1625 86.275) (width 0.2) (layer "B.Cu") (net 8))
 (segment (start 148.1625 86.275) (end 151.176471 86.275) (width 0.2) (layer "B.Cu") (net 8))
 (segment (start 144.1 86.9) (end 145.9875 86.9) (width 0.2) (layer "B.Cu") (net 8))
 (segment (start 136 86.1875) (end 138.9125 86.1875) (width 0.2) (layer "B.Cu") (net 8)))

